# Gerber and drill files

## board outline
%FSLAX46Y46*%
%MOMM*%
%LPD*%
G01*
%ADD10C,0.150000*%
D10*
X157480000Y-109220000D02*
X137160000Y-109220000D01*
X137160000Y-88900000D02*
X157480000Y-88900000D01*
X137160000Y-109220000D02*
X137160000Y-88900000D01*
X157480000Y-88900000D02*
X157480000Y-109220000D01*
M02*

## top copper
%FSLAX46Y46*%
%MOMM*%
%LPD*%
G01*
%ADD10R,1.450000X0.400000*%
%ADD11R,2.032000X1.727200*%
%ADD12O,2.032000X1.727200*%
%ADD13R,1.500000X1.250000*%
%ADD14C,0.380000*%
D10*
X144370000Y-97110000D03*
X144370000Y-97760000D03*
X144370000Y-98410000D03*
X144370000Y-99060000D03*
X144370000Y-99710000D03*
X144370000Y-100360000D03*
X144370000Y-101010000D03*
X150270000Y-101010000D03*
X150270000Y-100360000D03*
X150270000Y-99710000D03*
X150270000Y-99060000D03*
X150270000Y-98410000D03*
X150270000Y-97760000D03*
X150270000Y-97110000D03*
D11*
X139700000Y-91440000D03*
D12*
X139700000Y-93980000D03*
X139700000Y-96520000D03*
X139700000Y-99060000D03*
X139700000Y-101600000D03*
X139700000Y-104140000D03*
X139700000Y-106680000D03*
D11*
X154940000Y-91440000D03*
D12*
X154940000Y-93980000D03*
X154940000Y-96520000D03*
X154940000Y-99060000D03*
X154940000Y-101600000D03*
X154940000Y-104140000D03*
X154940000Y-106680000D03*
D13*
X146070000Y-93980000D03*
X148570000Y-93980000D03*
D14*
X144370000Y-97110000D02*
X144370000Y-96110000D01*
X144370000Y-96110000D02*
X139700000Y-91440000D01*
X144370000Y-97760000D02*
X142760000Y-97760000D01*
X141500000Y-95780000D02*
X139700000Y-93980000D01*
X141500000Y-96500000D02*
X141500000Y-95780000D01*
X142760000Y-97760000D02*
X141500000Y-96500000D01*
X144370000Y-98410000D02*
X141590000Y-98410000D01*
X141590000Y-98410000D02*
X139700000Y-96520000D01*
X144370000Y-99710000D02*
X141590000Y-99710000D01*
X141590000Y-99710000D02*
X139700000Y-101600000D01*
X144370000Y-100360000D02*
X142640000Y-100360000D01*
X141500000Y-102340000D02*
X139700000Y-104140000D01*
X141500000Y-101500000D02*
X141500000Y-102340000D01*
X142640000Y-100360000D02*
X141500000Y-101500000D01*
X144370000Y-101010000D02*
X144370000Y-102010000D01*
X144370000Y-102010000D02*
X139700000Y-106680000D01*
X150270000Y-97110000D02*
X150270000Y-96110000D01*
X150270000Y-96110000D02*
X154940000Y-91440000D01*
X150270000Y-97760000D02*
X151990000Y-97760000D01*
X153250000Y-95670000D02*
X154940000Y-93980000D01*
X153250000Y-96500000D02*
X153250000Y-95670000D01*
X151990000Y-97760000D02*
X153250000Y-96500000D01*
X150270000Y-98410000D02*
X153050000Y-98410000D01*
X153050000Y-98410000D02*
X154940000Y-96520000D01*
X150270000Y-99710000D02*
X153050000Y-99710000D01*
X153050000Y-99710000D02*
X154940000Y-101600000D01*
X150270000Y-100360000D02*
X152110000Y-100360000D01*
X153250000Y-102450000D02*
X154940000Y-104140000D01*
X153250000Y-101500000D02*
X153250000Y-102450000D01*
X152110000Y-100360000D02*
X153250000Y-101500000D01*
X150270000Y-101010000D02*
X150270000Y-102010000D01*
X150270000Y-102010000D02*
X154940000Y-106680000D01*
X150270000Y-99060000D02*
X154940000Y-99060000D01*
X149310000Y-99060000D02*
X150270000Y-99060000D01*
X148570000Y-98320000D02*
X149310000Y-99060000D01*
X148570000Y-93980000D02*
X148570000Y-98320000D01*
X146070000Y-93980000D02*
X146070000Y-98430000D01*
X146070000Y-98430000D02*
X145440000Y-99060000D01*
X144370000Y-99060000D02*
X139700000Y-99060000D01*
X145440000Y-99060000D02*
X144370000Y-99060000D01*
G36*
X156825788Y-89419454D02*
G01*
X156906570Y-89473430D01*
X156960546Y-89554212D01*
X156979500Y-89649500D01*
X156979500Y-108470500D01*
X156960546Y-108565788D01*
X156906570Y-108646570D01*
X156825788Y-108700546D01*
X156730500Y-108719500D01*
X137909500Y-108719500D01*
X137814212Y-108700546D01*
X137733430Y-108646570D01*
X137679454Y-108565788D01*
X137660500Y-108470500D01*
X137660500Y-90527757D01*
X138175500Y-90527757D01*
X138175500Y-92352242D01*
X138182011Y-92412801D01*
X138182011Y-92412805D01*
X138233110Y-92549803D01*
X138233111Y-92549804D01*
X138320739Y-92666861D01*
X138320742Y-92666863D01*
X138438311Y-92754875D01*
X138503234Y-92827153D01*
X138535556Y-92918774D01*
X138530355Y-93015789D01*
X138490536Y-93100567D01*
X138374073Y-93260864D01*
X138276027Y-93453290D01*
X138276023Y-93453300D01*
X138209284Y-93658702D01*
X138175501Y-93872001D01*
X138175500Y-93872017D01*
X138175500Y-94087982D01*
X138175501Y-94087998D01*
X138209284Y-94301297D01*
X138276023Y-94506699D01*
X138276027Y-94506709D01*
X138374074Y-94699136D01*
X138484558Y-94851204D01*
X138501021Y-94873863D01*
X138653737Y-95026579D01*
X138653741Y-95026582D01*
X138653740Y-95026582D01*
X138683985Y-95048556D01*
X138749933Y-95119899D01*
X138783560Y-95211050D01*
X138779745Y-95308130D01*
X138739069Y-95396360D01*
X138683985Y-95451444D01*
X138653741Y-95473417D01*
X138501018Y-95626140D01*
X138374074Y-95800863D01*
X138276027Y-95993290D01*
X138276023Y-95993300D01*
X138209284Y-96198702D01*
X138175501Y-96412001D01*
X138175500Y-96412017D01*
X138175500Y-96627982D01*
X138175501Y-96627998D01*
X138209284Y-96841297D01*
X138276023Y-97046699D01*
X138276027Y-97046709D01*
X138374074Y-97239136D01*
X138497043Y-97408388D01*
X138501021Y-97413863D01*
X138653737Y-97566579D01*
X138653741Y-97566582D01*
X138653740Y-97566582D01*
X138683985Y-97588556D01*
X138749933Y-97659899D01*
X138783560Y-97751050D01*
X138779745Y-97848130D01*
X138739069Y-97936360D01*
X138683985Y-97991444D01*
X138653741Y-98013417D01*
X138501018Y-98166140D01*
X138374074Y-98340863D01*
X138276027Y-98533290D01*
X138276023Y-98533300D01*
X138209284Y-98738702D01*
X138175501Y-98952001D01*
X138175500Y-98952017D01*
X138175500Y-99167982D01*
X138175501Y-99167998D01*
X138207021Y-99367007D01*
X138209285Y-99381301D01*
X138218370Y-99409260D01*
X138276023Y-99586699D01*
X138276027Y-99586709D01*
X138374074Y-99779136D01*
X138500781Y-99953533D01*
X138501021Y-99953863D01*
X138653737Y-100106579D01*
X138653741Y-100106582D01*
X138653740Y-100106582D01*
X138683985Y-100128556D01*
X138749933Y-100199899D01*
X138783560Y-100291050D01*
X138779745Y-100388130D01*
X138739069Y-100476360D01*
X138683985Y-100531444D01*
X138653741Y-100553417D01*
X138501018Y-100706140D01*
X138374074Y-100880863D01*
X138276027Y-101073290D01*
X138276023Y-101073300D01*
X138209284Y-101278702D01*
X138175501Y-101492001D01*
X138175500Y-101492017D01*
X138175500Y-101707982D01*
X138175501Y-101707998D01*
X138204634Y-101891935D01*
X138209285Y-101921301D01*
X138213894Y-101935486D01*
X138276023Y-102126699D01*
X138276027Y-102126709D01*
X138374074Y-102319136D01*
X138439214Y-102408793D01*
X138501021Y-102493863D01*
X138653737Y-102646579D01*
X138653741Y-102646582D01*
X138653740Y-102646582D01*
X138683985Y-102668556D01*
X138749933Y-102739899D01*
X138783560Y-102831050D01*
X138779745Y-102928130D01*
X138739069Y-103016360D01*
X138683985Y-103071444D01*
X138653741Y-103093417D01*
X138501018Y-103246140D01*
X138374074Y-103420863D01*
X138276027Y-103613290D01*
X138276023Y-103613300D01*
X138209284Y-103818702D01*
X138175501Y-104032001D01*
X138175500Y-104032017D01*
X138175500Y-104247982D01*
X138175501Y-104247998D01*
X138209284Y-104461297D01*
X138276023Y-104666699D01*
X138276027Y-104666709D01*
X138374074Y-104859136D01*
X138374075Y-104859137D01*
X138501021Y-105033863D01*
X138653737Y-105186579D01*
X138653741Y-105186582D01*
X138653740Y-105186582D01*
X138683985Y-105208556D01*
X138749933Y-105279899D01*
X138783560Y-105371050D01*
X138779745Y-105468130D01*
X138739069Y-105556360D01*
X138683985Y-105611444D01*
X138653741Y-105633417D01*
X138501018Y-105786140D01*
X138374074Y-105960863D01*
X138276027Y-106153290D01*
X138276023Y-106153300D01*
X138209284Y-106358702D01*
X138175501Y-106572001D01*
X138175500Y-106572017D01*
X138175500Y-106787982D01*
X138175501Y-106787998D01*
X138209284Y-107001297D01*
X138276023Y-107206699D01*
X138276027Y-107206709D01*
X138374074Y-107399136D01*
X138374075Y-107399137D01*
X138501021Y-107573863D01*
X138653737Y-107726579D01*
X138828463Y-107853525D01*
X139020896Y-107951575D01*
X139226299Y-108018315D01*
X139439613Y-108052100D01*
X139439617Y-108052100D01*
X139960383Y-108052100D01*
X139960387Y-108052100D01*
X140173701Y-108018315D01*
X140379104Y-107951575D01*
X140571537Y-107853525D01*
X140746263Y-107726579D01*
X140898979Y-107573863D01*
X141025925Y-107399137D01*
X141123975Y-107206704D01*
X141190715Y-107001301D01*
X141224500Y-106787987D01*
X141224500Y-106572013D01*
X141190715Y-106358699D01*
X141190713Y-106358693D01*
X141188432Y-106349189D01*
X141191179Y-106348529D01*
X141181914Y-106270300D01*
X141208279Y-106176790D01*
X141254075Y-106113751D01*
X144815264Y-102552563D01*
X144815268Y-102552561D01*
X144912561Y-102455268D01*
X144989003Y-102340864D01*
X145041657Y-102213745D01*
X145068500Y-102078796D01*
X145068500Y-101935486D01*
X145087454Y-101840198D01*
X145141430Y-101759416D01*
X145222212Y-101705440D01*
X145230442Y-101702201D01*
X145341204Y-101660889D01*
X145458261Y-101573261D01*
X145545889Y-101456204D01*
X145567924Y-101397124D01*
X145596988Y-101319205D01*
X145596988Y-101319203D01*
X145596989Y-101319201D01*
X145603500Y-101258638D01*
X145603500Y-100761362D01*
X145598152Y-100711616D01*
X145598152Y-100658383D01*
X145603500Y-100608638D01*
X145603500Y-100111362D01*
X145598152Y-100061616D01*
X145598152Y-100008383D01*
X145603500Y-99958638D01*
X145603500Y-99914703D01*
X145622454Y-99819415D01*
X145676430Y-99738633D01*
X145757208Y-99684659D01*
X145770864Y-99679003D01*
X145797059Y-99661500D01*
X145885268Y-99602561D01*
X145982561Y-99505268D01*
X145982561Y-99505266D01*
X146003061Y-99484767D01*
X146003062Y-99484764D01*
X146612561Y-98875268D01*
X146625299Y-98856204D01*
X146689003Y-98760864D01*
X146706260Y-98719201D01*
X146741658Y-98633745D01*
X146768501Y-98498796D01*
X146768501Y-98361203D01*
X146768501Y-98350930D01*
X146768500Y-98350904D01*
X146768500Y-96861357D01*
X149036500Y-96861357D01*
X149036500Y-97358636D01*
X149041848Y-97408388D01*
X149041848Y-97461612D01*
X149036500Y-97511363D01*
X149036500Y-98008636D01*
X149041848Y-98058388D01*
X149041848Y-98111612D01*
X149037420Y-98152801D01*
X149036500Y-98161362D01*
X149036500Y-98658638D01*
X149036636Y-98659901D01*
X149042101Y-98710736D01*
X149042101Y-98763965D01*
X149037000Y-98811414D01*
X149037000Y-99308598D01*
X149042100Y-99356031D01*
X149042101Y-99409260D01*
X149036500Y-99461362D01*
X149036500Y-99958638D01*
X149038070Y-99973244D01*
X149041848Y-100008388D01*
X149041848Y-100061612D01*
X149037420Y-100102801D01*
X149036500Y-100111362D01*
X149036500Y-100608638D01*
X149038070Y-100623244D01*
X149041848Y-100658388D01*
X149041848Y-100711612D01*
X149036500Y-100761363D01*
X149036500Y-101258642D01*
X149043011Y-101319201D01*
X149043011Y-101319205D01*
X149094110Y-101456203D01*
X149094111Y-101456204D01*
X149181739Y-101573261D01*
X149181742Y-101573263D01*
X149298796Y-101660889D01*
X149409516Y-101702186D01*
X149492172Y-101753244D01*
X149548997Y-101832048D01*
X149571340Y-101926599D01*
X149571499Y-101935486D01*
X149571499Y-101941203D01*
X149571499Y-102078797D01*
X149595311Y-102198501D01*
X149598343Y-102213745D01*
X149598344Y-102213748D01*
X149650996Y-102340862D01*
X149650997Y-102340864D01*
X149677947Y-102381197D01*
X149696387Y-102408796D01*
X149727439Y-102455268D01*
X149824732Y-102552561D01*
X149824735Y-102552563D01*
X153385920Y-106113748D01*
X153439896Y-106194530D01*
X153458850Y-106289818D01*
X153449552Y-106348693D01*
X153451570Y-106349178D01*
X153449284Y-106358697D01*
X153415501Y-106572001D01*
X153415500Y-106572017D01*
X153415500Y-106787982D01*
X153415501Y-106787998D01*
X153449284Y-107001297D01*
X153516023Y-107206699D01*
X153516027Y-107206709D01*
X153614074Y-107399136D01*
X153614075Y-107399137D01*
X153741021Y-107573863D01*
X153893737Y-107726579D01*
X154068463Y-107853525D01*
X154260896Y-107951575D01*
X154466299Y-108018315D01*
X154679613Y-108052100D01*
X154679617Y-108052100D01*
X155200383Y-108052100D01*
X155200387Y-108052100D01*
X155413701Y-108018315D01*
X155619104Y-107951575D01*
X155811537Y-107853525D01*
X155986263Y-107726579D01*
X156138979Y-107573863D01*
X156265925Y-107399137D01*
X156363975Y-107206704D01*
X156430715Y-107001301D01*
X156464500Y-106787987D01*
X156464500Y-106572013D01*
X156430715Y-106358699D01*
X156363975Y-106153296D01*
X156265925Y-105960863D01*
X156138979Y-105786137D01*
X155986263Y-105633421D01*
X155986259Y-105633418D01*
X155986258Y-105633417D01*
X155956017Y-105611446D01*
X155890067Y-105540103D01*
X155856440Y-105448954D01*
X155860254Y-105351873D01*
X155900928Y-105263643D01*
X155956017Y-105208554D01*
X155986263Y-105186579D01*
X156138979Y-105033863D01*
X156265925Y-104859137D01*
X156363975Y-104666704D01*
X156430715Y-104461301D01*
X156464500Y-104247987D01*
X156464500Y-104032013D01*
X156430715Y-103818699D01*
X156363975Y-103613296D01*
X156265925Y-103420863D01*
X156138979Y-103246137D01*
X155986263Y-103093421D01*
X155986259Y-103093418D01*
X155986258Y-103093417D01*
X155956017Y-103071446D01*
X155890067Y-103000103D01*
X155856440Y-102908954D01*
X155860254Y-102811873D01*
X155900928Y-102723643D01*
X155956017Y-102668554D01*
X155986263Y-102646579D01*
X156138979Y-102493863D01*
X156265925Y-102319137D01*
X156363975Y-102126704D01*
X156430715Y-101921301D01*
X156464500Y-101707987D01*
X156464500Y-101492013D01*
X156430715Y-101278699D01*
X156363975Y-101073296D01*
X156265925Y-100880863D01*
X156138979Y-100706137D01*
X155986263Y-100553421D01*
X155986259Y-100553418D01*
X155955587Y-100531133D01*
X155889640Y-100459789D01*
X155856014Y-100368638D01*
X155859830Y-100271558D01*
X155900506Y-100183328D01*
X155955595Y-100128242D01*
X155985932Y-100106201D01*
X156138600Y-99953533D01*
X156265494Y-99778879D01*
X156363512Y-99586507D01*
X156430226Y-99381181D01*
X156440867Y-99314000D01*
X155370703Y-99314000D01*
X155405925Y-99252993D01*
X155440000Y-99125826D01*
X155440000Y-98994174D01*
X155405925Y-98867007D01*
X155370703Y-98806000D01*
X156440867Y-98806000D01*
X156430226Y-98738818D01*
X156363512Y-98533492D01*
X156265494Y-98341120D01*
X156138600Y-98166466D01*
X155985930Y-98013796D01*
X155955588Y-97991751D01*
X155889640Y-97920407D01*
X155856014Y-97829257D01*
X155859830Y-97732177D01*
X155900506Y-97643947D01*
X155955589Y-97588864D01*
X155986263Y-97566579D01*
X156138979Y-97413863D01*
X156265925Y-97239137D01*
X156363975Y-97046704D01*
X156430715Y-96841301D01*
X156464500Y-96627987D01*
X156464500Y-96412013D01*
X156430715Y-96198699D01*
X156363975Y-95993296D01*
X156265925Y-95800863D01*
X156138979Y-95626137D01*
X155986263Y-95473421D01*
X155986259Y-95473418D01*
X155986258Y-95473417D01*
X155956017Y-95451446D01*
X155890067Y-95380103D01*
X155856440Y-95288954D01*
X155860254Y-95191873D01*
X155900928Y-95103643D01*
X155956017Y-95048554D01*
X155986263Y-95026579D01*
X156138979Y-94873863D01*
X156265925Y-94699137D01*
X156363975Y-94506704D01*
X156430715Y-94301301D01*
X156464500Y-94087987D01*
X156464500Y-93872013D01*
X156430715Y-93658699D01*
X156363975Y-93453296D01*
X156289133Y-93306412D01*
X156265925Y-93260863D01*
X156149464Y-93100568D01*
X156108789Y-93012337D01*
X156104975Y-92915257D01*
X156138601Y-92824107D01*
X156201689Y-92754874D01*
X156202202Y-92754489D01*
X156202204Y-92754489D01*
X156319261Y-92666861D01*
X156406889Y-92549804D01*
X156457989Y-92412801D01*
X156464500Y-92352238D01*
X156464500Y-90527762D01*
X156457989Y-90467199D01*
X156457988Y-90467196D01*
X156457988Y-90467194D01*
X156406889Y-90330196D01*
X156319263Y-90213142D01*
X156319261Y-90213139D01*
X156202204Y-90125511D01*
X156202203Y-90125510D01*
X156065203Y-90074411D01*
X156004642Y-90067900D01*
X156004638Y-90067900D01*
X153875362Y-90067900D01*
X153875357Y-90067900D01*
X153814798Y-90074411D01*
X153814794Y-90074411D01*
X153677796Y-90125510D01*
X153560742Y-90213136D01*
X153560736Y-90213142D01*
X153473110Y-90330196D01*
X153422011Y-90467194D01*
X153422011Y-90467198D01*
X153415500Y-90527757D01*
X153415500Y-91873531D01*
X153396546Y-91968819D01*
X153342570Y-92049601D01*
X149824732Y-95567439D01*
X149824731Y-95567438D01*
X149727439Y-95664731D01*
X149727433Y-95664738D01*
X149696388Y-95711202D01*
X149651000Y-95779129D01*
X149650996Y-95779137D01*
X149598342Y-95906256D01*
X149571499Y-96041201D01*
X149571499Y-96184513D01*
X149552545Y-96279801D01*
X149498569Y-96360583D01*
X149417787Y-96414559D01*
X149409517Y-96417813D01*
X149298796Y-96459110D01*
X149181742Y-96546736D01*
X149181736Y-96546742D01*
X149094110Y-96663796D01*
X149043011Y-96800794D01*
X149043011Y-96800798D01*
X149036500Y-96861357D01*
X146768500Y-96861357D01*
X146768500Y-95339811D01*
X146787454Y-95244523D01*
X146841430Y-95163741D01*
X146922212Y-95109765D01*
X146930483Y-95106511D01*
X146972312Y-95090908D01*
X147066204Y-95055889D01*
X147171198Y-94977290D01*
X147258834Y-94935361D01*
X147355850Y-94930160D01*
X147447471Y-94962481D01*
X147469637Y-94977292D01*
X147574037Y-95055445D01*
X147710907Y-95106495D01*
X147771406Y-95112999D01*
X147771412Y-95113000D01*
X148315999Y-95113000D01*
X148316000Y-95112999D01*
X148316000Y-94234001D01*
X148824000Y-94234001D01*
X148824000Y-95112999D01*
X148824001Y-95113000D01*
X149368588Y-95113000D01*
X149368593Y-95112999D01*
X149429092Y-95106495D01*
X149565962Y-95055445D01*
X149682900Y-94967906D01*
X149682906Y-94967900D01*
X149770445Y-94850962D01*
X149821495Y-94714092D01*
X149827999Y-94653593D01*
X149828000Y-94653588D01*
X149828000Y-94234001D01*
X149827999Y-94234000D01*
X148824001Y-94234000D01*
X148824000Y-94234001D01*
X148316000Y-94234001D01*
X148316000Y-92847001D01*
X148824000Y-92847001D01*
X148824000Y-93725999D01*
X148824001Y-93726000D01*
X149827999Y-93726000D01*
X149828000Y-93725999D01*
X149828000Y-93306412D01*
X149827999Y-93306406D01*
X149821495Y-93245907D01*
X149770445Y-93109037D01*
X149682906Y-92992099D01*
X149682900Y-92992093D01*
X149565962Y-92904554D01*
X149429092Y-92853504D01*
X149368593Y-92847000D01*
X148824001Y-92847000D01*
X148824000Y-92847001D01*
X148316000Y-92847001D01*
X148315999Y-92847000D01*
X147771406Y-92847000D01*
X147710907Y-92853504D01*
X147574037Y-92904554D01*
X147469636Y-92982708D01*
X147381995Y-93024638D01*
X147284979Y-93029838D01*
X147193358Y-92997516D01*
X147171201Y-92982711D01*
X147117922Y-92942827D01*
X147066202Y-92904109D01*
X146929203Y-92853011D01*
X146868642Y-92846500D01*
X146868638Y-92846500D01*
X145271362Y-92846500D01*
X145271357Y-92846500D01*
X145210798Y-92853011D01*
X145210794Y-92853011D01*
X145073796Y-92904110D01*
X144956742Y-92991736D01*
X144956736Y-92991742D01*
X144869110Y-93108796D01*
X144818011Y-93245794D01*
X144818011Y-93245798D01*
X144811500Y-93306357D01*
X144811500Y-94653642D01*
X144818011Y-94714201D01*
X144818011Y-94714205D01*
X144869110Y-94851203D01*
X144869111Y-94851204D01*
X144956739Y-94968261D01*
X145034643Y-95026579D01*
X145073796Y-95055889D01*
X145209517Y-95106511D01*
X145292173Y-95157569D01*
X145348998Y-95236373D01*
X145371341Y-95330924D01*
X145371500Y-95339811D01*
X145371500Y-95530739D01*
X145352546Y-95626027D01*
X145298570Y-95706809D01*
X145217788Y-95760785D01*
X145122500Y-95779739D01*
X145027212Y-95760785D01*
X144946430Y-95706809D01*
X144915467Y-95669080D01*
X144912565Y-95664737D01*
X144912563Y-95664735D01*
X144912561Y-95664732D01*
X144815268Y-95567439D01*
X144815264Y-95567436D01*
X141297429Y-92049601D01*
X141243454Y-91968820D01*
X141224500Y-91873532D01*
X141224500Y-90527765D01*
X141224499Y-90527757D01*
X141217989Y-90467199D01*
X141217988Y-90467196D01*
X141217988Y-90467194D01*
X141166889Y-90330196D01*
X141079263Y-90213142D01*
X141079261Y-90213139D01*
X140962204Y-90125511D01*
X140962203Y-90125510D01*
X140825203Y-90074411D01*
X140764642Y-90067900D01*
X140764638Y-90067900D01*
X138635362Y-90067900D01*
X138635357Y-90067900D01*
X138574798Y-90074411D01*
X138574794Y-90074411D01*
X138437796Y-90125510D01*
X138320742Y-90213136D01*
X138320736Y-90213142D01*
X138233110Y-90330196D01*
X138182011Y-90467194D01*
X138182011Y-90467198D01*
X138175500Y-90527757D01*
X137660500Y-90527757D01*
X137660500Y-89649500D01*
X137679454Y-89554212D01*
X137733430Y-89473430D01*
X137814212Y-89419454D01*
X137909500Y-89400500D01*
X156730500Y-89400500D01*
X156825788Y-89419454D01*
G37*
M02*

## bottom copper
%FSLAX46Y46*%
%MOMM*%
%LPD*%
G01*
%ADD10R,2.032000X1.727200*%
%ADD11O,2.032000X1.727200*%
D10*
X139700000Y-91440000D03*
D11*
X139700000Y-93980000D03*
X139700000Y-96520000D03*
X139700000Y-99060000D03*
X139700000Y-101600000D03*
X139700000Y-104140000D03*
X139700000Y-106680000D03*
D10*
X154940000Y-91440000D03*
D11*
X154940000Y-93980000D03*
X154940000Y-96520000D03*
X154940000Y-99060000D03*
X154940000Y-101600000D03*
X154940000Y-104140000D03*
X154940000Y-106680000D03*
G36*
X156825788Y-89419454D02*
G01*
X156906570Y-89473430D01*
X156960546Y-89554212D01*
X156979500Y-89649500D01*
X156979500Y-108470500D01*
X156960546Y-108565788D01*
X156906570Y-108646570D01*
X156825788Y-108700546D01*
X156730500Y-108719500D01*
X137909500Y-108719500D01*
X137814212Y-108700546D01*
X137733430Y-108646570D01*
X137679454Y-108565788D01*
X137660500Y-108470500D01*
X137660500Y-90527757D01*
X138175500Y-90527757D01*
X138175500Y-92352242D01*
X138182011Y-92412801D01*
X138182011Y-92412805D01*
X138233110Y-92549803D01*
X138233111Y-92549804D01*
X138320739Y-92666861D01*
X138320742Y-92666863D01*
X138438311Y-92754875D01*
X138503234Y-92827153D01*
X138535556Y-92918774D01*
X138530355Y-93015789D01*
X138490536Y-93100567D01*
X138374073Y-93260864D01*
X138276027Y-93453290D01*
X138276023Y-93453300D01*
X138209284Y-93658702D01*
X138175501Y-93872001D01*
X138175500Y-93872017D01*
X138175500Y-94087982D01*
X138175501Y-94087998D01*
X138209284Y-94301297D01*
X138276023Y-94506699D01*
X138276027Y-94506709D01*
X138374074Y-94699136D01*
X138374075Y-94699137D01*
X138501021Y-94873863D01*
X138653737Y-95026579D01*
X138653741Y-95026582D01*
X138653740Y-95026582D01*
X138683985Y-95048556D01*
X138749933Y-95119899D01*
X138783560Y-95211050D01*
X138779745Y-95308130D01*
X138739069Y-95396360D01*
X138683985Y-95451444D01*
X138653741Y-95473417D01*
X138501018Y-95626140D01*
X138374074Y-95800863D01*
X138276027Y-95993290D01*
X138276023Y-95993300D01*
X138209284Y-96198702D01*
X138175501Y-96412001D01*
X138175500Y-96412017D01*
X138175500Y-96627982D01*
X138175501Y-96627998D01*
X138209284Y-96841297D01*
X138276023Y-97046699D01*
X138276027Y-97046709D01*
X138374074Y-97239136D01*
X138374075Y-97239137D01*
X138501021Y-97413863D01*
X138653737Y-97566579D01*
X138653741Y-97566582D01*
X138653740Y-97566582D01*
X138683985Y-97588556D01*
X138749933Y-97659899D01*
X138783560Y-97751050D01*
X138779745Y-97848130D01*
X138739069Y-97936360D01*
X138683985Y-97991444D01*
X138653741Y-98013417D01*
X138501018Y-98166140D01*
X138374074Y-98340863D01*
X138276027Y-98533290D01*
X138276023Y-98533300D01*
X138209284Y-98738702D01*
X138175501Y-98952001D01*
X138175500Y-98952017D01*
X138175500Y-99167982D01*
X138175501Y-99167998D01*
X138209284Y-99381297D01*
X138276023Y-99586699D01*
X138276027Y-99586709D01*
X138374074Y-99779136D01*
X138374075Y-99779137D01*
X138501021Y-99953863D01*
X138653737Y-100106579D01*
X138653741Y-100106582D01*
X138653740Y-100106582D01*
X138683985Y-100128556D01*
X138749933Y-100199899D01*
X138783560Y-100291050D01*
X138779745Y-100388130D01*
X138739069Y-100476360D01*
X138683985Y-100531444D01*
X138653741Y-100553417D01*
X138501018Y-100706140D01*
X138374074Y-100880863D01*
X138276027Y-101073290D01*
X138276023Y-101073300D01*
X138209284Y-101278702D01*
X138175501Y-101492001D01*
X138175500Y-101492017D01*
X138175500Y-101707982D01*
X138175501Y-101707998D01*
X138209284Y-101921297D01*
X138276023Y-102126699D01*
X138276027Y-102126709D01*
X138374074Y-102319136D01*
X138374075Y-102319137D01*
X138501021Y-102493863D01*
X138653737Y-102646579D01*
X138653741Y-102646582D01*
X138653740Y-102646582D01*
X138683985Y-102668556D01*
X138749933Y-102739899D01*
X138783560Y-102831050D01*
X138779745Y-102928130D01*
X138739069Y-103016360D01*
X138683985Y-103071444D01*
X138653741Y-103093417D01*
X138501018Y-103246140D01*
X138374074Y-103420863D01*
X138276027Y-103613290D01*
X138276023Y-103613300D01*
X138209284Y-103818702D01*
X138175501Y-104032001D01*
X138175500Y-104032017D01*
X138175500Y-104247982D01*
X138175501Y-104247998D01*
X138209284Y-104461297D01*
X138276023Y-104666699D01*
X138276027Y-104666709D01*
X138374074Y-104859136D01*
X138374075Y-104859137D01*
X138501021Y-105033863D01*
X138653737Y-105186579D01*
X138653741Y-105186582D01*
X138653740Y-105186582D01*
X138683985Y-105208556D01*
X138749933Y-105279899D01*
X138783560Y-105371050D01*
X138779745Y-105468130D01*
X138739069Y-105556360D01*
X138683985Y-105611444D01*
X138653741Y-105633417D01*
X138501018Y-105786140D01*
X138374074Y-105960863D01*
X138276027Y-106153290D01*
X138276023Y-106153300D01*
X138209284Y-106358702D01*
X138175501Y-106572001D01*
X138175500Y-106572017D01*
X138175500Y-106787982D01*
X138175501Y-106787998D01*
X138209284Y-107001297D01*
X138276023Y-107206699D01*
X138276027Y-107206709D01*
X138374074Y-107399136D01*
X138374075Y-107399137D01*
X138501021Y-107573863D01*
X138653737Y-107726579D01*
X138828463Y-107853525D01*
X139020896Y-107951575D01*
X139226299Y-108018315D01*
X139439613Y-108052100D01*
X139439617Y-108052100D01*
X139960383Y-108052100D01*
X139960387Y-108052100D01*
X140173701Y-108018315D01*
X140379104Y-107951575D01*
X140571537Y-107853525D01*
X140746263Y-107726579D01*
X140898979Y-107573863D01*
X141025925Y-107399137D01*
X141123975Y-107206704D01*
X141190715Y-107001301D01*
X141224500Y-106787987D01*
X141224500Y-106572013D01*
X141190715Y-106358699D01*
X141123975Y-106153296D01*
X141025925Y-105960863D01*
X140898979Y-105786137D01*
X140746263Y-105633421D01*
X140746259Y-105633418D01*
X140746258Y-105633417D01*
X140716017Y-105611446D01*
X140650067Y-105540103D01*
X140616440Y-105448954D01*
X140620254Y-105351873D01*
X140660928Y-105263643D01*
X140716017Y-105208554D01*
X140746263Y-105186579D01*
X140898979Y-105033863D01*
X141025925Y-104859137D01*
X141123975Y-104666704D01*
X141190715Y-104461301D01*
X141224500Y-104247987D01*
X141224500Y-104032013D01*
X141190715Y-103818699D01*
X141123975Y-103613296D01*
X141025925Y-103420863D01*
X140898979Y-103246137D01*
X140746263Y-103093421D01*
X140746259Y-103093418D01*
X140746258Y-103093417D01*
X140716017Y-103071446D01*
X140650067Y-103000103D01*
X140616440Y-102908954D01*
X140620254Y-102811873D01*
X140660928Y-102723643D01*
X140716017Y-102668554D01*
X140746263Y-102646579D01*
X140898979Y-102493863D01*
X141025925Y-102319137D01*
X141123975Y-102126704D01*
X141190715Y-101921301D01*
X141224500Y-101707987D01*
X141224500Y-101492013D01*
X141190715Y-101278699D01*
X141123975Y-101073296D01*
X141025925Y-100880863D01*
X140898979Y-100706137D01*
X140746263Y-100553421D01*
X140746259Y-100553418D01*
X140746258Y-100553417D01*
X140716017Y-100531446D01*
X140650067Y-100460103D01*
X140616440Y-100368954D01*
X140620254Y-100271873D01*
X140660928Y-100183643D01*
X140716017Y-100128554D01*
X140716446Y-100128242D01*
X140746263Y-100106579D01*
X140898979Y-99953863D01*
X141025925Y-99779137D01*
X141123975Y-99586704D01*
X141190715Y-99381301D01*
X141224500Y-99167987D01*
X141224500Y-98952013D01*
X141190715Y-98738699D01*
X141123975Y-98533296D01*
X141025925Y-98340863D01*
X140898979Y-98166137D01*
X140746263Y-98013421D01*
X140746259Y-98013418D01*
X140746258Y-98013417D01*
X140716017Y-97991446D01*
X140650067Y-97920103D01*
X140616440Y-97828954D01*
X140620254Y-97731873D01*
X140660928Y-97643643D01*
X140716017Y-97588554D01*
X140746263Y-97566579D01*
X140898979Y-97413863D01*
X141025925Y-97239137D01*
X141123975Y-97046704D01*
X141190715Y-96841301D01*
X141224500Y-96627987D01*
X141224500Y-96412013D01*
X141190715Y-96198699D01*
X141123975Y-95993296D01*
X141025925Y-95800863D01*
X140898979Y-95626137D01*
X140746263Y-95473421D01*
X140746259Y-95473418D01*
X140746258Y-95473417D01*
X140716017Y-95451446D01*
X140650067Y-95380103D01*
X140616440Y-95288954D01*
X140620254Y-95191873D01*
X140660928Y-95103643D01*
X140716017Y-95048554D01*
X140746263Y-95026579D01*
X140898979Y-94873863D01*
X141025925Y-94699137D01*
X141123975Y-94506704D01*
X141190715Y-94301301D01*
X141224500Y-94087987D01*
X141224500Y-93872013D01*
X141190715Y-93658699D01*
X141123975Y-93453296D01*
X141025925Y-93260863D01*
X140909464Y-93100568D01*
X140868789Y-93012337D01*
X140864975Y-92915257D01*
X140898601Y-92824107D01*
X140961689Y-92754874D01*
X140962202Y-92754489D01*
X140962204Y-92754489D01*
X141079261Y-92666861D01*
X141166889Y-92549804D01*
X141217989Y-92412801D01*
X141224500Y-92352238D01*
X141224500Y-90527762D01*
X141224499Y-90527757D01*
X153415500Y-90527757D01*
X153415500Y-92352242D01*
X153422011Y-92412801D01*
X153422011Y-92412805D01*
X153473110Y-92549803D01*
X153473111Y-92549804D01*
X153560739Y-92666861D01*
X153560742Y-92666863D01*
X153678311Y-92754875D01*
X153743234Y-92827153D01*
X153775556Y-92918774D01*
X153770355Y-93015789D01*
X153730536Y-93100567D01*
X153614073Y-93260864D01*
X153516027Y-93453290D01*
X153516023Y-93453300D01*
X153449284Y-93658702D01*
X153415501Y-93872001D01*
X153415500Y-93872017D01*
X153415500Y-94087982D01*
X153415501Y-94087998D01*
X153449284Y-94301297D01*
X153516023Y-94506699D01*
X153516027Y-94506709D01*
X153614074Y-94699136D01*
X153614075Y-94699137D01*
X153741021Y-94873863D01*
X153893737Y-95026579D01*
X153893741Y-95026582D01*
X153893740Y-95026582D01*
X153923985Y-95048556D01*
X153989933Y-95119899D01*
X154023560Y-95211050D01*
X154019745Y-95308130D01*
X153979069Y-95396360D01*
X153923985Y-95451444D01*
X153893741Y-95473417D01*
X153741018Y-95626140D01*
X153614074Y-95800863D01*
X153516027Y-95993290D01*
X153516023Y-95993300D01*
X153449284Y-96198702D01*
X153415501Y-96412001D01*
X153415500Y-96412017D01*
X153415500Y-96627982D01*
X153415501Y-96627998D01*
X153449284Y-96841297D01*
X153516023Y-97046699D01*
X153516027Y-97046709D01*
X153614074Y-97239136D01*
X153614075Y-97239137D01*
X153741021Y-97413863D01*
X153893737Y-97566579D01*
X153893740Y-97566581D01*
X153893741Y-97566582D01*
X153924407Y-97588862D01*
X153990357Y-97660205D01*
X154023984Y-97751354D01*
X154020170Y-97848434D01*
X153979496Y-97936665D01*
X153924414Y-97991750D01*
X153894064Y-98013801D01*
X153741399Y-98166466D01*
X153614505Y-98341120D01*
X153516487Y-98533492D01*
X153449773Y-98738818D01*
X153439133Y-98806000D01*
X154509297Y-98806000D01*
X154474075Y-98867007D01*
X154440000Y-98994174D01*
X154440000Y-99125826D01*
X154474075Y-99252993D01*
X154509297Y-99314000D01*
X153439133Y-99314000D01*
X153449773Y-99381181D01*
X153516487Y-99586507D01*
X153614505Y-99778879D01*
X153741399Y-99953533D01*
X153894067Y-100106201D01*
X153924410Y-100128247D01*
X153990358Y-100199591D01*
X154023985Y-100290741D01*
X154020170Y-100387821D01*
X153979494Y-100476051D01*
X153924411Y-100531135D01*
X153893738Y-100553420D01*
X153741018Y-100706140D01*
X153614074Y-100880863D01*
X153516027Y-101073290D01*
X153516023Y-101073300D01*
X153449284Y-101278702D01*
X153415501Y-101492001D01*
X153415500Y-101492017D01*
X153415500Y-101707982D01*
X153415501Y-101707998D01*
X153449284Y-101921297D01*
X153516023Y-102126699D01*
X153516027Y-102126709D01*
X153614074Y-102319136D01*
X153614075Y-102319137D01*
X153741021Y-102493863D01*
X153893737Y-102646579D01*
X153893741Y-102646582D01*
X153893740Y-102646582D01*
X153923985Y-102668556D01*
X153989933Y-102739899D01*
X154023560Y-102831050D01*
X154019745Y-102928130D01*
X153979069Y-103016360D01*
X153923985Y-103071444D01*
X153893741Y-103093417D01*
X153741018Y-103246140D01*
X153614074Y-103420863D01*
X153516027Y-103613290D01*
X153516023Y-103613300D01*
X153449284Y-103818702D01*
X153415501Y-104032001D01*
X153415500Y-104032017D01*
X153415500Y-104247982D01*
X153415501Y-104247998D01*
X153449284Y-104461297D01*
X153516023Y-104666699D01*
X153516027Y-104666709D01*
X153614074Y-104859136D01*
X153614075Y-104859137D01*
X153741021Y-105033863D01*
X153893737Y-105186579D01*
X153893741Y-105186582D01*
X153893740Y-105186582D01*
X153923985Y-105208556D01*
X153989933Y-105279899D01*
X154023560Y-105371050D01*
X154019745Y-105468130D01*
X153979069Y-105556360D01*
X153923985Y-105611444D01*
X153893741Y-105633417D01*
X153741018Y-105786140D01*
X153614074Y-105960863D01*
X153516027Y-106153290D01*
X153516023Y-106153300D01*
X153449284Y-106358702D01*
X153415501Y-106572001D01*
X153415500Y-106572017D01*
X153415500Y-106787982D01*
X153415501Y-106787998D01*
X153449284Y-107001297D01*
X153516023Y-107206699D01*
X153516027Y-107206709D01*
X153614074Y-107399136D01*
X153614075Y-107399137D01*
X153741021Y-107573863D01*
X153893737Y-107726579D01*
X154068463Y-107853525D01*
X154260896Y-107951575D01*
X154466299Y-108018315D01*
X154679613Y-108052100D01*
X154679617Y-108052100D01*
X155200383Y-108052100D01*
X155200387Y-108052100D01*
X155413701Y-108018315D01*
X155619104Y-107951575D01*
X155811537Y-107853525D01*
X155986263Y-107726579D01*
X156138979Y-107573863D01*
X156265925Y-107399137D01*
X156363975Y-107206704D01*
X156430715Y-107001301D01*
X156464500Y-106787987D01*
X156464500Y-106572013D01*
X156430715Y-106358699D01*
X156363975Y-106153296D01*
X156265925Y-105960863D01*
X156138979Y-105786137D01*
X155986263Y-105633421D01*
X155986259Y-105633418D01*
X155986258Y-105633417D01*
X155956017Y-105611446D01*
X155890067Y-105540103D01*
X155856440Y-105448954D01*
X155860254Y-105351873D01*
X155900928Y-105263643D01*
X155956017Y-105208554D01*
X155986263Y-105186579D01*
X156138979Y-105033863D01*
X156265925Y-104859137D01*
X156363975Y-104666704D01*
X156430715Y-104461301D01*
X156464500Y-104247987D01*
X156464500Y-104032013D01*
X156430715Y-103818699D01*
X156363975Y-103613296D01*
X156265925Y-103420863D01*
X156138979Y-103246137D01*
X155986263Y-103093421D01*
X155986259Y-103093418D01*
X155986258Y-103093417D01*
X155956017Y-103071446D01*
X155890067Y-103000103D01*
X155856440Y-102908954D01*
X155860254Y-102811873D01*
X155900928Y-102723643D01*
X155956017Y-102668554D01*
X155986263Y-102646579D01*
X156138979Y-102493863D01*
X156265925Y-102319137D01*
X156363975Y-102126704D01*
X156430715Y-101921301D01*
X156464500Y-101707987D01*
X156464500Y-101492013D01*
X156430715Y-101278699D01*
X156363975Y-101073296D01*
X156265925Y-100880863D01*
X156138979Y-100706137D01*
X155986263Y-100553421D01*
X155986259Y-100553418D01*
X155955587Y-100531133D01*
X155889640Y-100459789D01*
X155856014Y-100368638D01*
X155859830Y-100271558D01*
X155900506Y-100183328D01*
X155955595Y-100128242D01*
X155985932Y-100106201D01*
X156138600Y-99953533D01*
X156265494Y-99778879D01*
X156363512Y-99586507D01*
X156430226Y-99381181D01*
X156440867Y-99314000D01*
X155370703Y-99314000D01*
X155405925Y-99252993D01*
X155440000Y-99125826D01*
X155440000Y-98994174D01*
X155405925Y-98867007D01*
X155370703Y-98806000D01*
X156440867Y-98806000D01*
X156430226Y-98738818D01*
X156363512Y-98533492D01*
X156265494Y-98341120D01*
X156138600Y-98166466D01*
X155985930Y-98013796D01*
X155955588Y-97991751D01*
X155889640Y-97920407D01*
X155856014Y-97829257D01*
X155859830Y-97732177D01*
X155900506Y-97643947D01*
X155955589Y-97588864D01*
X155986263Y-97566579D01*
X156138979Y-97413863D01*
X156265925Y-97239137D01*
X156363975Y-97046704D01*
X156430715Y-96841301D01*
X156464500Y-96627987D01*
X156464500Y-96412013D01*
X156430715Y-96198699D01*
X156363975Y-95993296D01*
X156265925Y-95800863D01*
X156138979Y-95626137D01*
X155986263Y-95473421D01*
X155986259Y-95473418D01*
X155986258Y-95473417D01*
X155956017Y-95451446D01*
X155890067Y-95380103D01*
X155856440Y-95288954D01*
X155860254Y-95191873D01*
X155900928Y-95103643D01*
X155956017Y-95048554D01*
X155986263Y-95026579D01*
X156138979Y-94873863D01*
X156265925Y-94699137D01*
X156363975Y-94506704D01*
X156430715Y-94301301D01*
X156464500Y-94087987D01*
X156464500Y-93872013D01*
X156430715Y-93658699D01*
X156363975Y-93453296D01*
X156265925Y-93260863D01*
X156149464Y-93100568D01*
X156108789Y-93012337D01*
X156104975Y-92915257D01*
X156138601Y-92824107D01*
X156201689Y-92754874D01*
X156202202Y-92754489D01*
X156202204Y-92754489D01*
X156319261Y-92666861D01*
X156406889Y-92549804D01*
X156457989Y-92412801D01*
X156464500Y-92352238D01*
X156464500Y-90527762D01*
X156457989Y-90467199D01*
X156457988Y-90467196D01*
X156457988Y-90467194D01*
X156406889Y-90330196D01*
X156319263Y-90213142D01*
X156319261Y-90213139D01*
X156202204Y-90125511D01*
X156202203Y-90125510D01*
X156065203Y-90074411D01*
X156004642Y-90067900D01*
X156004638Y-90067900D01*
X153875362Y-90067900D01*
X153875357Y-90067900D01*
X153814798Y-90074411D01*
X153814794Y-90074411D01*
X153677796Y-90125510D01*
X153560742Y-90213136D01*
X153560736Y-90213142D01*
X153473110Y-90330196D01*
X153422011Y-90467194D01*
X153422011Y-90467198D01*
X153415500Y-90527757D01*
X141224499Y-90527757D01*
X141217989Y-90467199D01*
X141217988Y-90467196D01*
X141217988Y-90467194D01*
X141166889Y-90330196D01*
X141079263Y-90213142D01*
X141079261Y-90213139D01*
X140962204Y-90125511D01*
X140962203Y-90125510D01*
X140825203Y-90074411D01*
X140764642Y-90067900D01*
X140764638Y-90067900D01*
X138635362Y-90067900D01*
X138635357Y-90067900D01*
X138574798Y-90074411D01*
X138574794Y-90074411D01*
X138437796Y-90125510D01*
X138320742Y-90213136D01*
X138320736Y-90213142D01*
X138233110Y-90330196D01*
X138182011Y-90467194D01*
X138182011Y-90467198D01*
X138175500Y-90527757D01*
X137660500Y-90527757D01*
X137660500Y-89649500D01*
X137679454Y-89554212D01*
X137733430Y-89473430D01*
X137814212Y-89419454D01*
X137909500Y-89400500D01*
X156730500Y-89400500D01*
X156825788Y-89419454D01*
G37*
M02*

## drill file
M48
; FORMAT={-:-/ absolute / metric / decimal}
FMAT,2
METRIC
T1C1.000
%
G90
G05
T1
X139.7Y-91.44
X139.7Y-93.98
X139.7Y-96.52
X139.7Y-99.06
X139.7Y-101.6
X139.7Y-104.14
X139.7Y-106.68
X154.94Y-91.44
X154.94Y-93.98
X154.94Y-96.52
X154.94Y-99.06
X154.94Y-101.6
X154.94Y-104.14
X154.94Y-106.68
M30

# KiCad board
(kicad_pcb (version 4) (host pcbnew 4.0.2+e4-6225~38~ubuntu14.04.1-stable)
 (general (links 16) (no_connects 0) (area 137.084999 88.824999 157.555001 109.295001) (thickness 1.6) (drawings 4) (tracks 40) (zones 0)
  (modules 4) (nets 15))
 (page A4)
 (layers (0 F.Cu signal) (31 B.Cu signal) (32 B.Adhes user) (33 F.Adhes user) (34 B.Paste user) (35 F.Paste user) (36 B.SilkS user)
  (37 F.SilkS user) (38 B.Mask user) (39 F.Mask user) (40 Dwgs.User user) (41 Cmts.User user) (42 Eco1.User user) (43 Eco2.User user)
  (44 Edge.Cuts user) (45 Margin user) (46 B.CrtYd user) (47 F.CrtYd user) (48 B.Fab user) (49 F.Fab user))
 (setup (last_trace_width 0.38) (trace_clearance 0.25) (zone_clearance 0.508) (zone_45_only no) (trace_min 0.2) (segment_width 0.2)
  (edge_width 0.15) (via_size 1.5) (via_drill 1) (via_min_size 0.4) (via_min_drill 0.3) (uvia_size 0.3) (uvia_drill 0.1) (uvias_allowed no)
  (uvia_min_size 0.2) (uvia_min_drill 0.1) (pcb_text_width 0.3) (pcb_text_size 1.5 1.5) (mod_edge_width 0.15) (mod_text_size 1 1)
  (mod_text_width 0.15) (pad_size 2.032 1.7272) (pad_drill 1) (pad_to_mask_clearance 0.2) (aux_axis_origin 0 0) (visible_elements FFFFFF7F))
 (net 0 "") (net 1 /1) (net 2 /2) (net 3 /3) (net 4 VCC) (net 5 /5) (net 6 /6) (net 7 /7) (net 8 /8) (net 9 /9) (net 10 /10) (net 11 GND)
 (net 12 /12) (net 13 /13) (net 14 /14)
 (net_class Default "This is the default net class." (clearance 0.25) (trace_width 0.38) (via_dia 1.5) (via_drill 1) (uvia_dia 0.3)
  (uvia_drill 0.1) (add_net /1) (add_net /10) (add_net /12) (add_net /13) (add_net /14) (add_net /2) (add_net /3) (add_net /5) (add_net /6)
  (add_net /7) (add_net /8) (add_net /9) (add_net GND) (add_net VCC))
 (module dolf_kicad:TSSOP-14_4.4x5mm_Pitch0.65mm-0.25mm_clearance (layer F.Cu) (at 147.32 99.06)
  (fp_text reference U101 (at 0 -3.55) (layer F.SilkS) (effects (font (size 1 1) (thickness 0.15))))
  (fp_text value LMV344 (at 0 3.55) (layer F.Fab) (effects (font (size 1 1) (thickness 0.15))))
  (pad 1 smd rect (at -2.95 -1.95) (size 1.45 0.4) (layers F.Cu F.Paste F.Mask) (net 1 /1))
  (pad 2 smd rect (at -2.95 -1.3) (size 1.45 0.4) (layers F.Cu F.Paste F.Mask) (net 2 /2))
  (pad 3 smd rect (at -2.95 -0.65) (size 1.45 0.4) (layers F.Cu F.Paste F.Mask) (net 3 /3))
  (pad 4 smd rect (at -2.95 0) (size 1.45 0.4) (layers F.Cu F.Paste F.Mask) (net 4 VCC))
  (pad 5 smd rect (at -2.95 0.65) (size 1.45 0.4) (layers F.Cu F.Paste F.Mask) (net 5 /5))
  (pad 6 smd rect (at -2.95 1.3) (size 1.45 0.4) (layers F.Cu F.Paste F.Mask) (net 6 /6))
  (pad 7 smd rect (at -2.95 1.95) (size 1.45 0.4) (layers F.Cu F.Paste F.Mask) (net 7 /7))
  (pad 8 smd rect (at 2.95 1.95) (size 1.45 0.4) (layers F.Cu F.Paste F.Mask) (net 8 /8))
  (pad 9 smd rect (at 2.95 1.3) (size 1.45 0.4) (layers F.Cu F.Paste F.Mask) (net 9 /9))
  (pad 10 smd rect (at 2.95 0.65) (size 1.45 0.4) (layers F.Cu F.Paste F.Mask) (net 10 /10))
  (pad 11 smd rect (at 2.95 0) (size 1.45 0.4) (layers F.Cu F.Paste F.Mask) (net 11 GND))
  (pad 12 smd rect (at 2.95 -0.65) (size 1.45 0.4) (layers F.Cu F.Paste F.Mask) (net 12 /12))
  (pad 13 smd rect (at 2.95 -1.3) (size 1.45 0.4) (layers F.Cu F.Paste F.Mask) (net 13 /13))
  (pad 14 smd rect (at 2.95 -1.95) (size 1.45 0.4) (layers F.Cu F.Paste F.Mask) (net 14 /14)))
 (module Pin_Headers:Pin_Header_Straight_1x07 (layer F.Cu) (at 139.7 91.44)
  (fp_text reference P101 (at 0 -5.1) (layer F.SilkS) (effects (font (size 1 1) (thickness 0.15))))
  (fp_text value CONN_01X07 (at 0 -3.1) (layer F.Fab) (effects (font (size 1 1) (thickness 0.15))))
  (pad 1 thru_hole rect (at 0 0) (size 2.032 1.7272) (drill 1) (layers *.Cu *.Mask F.SilkS) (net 1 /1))
  (pad 2 thru_hole oval (at 0 2.54) (size 2.032 1.7272) (drill 1) (layers *.Cu *.Mask F.SilkS) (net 2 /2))
  (pad 3 thru_hole oval (at 0 5.08) (size 2.032 1.7272) (drill 1) (layers *.Cu *.Mask F.SilkS) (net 3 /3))
  (pad 4 thru_hole oval (at 0 7.62) (size 2.032 1.7272) (drill 1) (layers *.Cu *.Mask F.SilkS) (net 4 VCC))
  (pad 5 thru_hole oval (at 0 10.16) (size 2.032 1.7272) (drill 1) (layers *.Cu *.Mask F.SilkS) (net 5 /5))
  (pad 6 thru_hole oval (at 0 12.7) (size 2.032 1.7272) (drill 1) (layers *.Cu *.Mask F.SilkS) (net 6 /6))
  (pad 7 thru_hole oval (at 0 15.24) (size 2.032 1.7272) (drill 1) (layers *.Cu *.Mask F.SilkS) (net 7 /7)))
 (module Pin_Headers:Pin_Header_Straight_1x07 (layer F.Cu) (at 154.94 91.44)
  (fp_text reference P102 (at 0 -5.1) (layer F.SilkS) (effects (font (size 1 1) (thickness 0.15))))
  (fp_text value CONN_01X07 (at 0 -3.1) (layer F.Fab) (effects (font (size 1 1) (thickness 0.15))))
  (pad 1 thru_hole rect (at 0 0) (size 2.032 1.7272) (drill 1) (layers *.Cu *.Mask F.SilkS) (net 14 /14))
  (pad 2 thru_hole oval (at 0 2.54) (size 2.032 1.7272) (drill 1) (layers *.Cu *.Mask F.SilkS) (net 13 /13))
  (pad 3 thru_hole oval (at 0 5.08) (size 2.032 1.7272) (drill 1) (layers *.Cu *.Mask F.SilkS) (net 12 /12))
  (pad 4 thru_hole oval (at 0 7.62) (size 2.032 1.7272) (drill 1) (layers *.Cu *.Mask F.SilkS) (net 11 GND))
  (pad 5 thru_hole oval (at 0 10.16) (size 2.032 1.7272) (drill 1) (layers *.Cu *.Mask F.SilkS) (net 10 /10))
  (pad 6 thru_hole oval (at 0 12.7) (size 2.032 1.7272) (drill 1) (layers *.Cu *.Mask F.SilkS) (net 9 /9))
  (pad 7 thru_hole oval (at 0 15.24) (size 2.032 1.7272) (drill 1) (layers *.Cu *.Mask F.SilkS) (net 8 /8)))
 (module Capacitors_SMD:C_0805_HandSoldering (layer F.Cu) (at 147.32 93.98)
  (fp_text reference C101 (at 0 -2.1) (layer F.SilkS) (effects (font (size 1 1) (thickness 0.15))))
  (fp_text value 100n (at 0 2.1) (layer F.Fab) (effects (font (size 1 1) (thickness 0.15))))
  (pad 1 smd rect (at -1.25 0) (size 1.5 1.25) (layers F.Cu F.Paste F.Mask) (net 4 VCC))
  (pad 2 smd rect (at 1.25 0) (size 1.5 1.25) (layers F.Cu F.Paste F.Mask) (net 11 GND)))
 (gr_line (start 157.48 109.22) (end 137.16 109.22) (angle 90) (layer Edge.Cuts) (width 0.15))
 (gr_line (start 137.16 88.9) (end 157.48 88.9) (angle 90) (layer Edge.Cuts) (width 0.15))
 (gr_line (start 137.16 109.22) (end 137.16 88.9) (angle 90) (layer Edge.Cuts) (width 0.15))
 (gr_line (start 157.48 88.9) (end 157.48 109.22) (angle 90) (layer Edge.Cuts) (width 0.15))
 (segment (start 144.37 97.11) (end 144.37 96.11) (width 0.38) (layer F.Cu) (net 1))
 (segment (start 144.37 96.11) (end 139.7 91.44) (width 0.38) (layer F.Cu) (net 1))
 (segment (start 144.37 97.76) (end 142.76 97.76) (width 0.38) (layer F.Cu) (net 2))
 (segment (start 141.5 95.78) (end 139.7 93.98) (width 0.38) (layer F.Cu) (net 2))
 (segment (start 141.5 96.5) (end 141.5 95.78) (width 0.38) (layer F.Cu) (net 2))
 (segment (start 142.76 97.76) (end 141.5 96.5) (width 0.38) (layer F.Cu) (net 2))
 (segment (start 144.37 98.41) (end 141.59 98.41) (width 0.38) (layer F.Cu) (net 3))
 (segment (start 141.59 98.41) (end 139.7 96.52) (width 0.38) (layer F.Cu) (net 3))
 (segment (start 144.37 99.71) (end 141.59 99.71) (width 0.38) (layer F.Cu) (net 5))
 (segment (start 141.59 99.71) (end 139.7 101.6) (width 0.38) (layer F.Cu) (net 5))
 (segment (start 144.37 100.36) (end 142.64 100.36) (width 0.38) (layer F.Cu) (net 6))
 (segment (start 141.5 102.34) (end 139.7 104.14) (width 0.38) (layer F.Cu) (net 6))
 (segment (start 141.5 101.5) (end 141.5 102.34) (width 0.38) (layer F.Cu) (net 6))
 (segment (start 142.64 100.36) (end 141.5 101.5) (width 0.38) (layer F.Cu) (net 6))
 (segment (start 144.37 101.01) (end 144.37 102.01) (width 0.38) (layer F.Cu) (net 7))
 (segment (start 144.37 102.01) (end 139.7 106.68) (width 0.38) (layer F.Cu) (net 7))
 (segment (start 150.27 97.11) (end 150.27 96.11) (width 0.38) (layer F.Cu) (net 14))
 (segment (start 150.27 96.11) (end 154.94 91.44) (width 0.38) (layer F.Cu) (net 14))
 (segment (start 150.27 97.76) (end 151.99 97.76) (width 0.38) (layer F.Cu) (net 13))
 (segment (start 153.25 95.67) (end 154.94 93.98) (width 0.38) (layer F.Cu) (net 13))
 (segment (start 153.25 96.5) (end 153.25 95.67) (width 0.38) (layer F.Cu) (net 13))
 (segment (start 151.99 97.76) (end 153.25 96.5) (width 0.38) (layer F.Cu) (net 13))
 (segment (start 150.27 98.41) (end 153.05 98.41) (width 0.38) (layer F.Cu) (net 12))
 (segment (start 153.05 98.41) (end 154.94 96.52) (width 0.38) (layer F.Cu) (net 12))
 (segment (start 150.27 99.71) (end 153.05 99.71) (width 0.38) (layer F.Cu) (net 10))
 (segment (start 153.05 99.71) (end 154.94 101.6) (width 0.38) (layer F.Cu) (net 10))
 (segment (start 150.27 100.36) (end 152.11 100.36) (width 0.38) (layer F.Cu) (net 9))
 (segment (start 153.25 102.45) (end 154.94 104.14) (width 0.38) (layer F.Cu) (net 9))
 (segment (start 153.25 101.5) (end 153.25 102.45) (width 0.38) (layer F.Cu) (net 9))
 (segment (start 152.11 100.36) (end 153.25 101.5) (width 0.38) (layer F.Cu) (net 9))
 (segment (start 150.27 101.01) (end 150.27 102.01) (width 0.38) (layer F.Cu) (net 8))
 (segment (start 150.27 102.01) (end 154.94 106.68) (width 0.38) (layer F.Cu) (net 8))
 (segment (start 150.27 99.06) (end 154.94 99.06) (width 0.38) (layer F.Cu) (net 11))
 (segment (start 149.31 99.06) (end 150.27 99.06) (width 0.38) (layer F.Cu) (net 11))
 (segment (start 148.57 98.32) (end 149.31 99.06) (width 0.38) (layer F.Cu) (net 11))
 (segment (start 148.57 93.98) (end 148.57 98.32) (width 0.38) (layer F.Cu) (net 11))
 (segment (start 146.07 93.98) (end 146.07 98.43) (width 0.38) (layer F.Cu) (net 4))
 (segment (start 146.07 98.43) (end 145.44 99.06) (width 0.38) (layer F.Cu) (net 4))
 (segment (start 144.37 99.06) (end 139.7 99.06) (width 0.38) (layer F.Cu) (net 4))
 (segment (start 145.44 99.06) (end 144.37 99.06) (width 0.38) (layer F.Cu) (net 4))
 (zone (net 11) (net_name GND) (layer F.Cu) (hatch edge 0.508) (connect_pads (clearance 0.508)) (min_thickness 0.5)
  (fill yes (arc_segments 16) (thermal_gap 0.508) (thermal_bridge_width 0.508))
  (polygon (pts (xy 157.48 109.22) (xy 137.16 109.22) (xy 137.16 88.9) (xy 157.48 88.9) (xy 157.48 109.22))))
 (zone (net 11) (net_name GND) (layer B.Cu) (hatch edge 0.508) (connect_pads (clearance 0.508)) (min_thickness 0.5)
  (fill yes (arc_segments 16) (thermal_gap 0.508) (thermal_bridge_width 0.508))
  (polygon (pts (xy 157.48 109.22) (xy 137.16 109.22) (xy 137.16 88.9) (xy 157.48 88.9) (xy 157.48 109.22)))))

